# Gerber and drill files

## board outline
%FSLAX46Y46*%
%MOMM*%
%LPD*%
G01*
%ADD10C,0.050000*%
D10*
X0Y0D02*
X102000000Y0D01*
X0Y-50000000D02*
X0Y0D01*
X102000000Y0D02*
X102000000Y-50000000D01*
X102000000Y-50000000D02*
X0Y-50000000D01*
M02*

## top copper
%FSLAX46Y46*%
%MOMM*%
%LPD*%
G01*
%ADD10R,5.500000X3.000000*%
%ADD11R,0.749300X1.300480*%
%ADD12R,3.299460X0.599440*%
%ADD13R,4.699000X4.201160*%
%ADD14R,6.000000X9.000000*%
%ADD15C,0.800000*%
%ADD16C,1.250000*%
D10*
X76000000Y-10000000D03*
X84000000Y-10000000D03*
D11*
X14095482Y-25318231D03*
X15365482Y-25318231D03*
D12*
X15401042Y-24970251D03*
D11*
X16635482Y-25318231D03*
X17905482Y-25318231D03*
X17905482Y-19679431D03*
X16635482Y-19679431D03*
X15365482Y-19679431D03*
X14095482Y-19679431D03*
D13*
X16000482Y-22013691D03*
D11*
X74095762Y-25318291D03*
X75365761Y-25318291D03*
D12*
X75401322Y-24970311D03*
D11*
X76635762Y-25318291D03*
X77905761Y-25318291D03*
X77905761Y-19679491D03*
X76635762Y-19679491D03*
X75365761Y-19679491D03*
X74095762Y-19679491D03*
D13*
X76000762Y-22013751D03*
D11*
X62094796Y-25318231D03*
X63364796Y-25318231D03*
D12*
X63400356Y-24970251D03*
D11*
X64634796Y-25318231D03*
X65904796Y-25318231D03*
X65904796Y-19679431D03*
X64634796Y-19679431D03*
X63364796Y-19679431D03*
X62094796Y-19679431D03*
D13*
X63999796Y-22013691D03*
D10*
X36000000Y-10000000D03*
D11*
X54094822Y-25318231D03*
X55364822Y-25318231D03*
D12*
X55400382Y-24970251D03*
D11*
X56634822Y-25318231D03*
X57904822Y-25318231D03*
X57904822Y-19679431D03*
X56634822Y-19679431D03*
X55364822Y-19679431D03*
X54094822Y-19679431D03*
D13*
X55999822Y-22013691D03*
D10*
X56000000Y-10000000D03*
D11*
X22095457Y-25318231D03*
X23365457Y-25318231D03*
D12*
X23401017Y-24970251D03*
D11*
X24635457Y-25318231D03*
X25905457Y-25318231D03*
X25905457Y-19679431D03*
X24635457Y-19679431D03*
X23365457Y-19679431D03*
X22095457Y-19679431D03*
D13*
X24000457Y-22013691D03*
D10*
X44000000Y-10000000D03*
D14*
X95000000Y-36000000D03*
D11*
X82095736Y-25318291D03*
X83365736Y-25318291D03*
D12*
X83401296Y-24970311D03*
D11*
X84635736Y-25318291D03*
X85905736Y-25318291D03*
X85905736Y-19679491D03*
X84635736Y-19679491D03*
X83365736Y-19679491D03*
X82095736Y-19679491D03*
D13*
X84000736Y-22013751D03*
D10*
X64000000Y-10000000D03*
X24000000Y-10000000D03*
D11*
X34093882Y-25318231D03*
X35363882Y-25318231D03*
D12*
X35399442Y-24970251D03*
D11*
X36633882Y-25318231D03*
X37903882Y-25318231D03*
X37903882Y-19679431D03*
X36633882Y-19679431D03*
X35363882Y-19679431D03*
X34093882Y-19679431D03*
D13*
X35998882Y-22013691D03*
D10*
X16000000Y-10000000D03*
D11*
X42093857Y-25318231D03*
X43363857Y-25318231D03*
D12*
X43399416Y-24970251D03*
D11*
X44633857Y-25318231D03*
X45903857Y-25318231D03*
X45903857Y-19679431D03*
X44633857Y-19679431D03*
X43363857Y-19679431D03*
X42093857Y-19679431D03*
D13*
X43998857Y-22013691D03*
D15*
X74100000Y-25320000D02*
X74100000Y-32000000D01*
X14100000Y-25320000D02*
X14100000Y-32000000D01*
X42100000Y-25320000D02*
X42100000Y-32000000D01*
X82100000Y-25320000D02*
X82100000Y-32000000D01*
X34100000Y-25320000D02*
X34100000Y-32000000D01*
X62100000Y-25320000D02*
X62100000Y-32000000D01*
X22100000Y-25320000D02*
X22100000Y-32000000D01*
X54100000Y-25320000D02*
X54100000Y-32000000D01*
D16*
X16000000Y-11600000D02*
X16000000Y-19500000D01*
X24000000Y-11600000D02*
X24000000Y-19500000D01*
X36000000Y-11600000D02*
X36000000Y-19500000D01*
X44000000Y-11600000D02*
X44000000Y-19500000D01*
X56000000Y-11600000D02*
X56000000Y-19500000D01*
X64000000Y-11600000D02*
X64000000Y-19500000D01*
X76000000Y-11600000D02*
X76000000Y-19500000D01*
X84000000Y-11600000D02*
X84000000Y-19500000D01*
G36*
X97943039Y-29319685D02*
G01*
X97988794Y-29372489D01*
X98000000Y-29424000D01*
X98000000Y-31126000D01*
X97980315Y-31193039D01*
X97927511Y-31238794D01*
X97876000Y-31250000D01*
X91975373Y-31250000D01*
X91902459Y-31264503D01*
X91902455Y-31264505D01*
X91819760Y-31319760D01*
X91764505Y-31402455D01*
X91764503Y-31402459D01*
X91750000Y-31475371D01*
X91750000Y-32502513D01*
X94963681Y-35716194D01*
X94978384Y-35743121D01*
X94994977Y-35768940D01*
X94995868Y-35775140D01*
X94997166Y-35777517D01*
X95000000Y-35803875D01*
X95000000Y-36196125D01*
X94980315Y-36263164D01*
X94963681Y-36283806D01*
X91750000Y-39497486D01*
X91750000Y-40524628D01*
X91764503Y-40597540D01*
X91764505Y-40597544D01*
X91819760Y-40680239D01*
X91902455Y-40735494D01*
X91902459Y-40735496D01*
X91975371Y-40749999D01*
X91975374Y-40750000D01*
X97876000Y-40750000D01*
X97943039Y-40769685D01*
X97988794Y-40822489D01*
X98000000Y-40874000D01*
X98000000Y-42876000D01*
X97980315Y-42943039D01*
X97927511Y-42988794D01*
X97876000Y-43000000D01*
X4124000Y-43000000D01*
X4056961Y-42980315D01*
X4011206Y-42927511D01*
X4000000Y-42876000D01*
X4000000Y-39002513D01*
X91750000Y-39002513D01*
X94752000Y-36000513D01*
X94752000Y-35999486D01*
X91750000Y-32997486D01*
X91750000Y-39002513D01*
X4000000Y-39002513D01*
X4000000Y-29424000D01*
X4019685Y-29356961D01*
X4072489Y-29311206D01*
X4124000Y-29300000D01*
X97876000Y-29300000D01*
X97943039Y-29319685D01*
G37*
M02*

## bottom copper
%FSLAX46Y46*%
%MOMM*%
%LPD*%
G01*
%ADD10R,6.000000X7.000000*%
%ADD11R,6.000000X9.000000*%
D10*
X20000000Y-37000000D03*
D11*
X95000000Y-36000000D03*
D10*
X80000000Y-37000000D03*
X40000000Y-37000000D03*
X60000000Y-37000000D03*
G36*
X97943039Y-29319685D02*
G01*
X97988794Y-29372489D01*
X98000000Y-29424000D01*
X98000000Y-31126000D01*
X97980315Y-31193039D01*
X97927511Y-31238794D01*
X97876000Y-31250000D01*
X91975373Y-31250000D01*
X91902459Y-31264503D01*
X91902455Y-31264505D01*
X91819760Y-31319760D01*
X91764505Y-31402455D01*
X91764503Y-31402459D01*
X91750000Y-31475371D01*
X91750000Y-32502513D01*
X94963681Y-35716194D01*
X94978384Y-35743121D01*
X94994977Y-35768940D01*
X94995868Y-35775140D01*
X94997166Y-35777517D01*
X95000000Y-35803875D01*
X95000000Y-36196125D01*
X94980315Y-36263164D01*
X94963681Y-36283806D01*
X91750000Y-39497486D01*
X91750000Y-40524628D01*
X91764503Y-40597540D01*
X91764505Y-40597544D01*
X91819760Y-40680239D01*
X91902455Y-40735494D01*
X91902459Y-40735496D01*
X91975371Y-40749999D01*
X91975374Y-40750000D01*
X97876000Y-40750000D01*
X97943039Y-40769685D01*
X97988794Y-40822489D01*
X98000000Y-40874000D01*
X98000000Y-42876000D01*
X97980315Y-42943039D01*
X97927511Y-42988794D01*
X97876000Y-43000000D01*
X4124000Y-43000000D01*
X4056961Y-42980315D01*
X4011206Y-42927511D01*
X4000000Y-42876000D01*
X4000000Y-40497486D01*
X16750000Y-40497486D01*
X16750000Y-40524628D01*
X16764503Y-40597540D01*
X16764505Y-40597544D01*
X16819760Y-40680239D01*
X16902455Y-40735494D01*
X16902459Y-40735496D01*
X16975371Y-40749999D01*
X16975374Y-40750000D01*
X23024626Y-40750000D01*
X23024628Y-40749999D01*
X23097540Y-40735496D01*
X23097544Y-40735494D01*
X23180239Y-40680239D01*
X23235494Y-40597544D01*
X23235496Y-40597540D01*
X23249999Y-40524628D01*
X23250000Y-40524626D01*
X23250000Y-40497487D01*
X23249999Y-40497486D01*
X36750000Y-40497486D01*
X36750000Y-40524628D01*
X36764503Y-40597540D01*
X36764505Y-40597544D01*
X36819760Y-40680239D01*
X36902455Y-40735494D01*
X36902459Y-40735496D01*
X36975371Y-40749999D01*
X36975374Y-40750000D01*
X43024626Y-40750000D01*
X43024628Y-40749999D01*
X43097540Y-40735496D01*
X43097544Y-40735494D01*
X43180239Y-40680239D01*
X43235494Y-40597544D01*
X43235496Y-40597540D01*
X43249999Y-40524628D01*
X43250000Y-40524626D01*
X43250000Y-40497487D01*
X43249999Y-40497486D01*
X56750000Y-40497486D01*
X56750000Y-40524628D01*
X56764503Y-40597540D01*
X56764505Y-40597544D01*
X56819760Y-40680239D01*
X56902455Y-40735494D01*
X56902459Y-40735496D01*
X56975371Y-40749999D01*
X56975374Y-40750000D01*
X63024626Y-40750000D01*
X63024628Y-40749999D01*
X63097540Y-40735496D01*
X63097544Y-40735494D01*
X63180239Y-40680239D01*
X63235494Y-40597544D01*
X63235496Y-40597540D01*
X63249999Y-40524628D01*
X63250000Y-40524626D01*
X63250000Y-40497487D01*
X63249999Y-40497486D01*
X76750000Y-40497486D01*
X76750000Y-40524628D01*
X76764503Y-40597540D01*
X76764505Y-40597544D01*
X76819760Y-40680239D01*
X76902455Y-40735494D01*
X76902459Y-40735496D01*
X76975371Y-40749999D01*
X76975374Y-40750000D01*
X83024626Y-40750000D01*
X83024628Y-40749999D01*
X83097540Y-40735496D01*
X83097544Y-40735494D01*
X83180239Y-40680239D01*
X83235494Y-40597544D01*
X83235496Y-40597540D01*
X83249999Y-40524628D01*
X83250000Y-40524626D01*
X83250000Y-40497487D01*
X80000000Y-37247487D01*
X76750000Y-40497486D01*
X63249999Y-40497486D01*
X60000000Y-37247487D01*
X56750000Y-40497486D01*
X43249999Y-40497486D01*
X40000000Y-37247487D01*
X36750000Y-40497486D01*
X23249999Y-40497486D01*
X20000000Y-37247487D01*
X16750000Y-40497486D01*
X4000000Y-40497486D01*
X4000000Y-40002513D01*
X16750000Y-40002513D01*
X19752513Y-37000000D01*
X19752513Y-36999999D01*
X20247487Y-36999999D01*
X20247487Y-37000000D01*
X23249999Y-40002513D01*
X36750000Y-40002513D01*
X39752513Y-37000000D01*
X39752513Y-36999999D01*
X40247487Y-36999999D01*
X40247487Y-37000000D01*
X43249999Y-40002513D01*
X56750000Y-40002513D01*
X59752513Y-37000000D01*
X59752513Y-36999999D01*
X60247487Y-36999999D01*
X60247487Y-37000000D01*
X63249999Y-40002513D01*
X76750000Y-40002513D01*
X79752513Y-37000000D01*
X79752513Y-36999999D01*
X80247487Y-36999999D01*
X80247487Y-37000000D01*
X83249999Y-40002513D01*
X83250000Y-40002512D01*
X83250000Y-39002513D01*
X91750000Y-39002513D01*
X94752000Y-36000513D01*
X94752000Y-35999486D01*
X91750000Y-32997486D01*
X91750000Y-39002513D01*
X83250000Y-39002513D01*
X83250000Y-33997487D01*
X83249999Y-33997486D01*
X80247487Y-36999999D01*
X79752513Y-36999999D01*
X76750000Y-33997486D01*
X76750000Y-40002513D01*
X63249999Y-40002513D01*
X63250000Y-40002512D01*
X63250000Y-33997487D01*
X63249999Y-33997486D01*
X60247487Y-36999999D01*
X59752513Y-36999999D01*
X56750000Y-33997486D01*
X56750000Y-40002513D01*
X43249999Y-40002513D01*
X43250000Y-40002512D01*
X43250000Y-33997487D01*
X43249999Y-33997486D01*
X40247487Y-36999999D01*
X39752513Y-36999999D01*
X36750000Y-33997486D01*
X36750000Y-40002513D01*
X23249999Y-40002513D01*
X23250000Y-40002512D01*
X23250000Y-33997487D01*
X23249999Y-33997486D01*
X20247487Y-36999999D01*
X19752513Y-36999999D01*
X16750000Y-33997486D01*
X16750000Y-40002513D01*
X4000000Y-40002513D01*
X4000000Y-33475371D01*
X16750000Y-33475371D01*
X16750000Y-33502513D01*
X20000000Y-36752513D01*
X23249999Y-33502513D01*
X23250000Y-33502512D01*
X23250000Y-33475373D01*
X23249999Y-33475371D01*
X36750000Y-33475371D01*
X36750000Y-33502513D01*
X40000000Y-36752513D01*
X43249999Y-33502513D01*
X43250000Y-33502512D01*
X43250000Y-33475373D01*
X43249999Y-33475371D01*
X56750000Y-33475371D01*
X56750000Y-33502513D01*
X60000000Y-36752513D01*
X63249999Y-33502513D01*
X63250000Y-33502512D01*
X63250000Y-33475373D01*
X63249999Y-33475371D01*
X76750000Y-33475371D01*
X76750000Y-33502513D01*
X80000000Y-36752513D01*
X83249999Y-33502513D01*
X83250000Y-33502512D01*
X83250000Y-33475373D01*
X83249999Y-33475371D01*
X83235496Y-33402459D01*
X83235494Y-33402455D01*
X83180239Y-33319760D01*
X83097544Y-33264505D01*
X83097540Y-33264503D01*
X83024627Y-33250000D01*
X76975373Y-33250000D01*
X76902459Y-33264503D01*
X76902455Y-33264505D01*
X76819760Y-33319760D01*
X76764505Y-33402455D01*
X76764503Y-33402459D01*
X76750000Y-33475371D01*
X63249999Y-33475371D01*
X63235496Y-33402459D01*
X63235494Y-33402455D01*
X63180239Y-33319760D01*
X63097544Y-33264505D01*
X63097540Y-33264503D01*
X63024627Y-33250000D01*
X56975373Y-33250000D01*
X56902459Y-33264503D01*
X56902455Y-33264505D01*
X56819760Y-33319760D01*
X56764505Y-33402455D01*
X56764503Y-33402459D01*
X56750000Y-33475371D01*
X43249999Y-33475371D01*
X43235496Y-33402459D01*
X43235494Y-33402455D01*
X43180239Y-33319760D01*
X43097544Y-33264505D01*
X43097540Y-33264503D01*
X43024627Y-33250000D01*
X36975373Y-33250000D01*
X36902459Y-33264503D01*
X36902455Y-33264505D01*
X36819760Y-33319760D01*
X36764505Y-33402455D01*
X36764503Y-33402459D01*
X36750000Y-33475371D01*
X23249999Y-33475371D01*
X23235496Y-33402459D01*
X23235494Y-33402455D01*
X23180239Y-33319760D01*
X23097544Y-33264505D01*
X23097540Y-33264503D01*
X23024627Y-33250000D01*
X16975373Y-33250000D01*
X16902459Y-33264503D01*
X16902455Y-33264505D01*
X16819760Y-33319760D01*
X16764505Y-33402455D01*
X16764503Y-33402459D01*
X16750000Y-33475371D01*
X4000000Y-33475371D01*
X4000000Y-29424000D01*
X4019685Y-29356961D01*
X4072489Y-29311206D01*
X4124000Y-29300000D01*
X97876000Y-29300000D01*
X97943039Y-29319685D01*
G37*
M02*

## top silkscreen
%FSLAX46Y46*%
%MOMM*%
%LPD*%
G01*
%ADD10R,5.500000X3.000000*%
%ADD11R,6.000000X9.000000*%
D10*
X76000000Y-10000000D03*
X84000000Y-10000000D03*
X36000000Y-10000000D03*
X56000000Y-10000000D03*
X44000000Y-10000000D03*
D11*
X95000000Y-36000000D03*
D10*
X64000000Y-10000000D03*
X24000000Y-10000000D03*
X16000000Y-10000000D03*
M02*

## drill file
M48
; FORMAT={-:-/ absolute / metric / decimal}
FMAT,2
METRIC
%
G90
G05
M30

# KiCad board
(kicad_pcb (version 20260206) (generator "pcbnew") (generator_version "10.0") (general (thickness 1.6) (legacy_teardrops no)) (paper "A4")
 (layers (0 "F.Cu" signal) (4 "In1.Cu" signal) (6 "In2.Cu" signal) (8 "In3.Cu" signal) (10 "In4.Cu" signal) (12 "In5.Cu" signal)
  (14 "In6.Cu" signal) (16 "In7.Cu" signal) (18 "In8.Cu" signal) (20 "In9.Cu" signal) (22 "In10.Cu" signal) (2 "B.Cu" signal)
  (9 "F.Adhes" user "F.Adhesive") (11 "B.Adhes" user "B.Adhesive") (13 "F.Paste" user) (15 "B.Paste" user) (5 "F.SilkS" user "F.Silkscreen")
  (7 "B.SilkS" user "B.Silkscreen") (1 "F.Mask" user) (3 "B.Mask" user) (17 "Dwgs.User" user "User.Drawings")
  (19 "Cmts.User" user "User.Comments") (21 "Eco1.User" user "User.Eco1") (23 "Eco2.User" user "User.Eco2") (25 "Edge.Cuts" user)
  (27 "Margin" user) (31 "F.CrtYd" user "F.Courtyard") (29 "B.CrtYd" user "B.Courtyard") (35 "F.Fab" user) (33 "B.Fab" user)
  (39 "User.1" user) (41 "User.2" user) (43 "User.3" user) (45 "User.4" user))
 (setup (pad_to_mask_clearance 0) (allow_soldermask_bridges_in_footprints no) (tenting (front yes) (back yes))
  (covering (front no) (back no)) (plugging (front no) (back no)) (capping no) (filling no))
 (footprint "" (layer "F.Cu") (at 76 10)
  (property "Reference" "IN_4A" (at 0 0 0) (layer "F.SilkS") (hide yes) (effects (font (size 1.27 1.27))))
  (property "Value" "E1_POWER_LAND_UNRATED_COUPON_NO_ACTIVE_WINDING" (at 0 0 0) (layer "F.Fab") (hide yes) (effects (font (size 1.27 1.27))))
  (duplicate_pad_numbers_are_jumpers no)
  (pad "1" smd rect (at 0 0) (size 5.5 3)
   (layers "F.Cu" "F.Mask" "F.SilkS" "F.Adhes" "F.Paste" "F.CrtYd" "F.Fab") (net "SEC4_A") (thermal_bridge_angle 45)))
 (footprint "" (layer "F.Cu") (at 84 10)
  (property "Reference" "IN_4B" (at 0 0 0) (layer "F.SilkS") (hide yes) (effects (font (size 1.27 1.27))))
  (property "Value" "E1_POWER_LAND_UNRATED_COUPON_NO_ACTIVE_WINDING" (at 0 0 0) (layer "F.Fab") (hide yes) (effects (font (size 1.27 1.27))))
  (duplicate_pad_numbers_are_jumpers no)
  (pad "1" smd rect (at 0 0) (size 5.5 3)
   (layers "F.Cu" "F.Mask" "F.SilkS" "F.Adhes" "F.Paste" "F.CrtYd" "F.Fab") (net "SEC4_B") (thermal_bridge_angle 45)))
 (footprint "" (layer "F.Cu") (at 16 22.5)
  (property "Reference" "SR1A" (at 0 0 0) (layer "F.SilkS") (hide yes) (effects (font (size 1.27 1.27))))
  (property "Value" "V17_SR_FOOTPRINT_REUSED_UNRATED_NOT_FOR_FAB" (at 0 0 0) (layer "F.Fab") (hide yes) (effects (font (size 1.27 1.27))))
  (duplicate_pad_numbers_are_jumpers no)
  (pad "1" smd rect (at -1.904518 2.818231 90) (size 1.30048 0.7493) (layers "F.Cu" "F.Mask" "F.Paste") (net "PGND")
   (thermal_bridge_angle 45))
  (pad "2" smd rect (at -0.634518 2.818231 90) (size 1.30048 0.7493) (layers "F.Cu" "F.Mask" "F.Paste") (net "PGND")
   (thermal_bridge_angle 45))
  (pad "3" smd rect (at -0.598958 2.470251 90) (size 0.59944 3.29946) (layers "F.Cu" "F.Mask" "F.Paste") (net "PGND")
   (thermal_bridge_angle 45))
  (pad "3" smd rect (at 0.635482 2.818231 90) (size 1.30048 0.7493) (layers "F.Cu" "F.Mask" "F.Paste") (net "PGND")
   (thermal_bridge_angle 45))
  (pad "4" smd rect (at 1.905482 2.818231 90) (size 1.30048 0.7493) (layers "F.Cu" "F.Mask" "F.Paste") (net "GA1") (thermal_bridge_angle 45))
  (pad "5" smd rect (at 1.905482 -2.820569 270) (size 1.30048 0.7493) (layers "F.Cu" "F.Mask" "F.Paste") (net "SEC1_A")
   (thermal_bridge_angle 45))
  (pad "6" smd rect (at 0.635482 -2.820569 270) (size 1.30048 0.7493) (layers "F.Cu" "F.Mask" "F.Paste") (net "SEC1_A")
   (thermal_bridge_angle 45))
  (pad "7" smd rect (at -0.634518 -2.820569 270) (size 1.30048 0.7493) (layers "F.Cu" "F.Mask" "F.Paste") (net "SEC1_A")
   (thermal_bridge_angle 45))
  (pad "8" smd rect (at -1.904518 -2.820569 270) (size 1.30048 0.7493) (layers "F.Cu" "F.Mask" "F.Paste") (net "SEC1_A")
   (thermal_bridge_angle 45))
  (pad "8" smd rect (at 0.000482 -0.486309) (size 4.699 4.20116) (layers "F.Cu" "F.Mask" "F.Paste") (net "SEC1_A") (thermal_bridge_angle 45)))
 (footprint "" (layer "F.Cu") (at 76 22.5)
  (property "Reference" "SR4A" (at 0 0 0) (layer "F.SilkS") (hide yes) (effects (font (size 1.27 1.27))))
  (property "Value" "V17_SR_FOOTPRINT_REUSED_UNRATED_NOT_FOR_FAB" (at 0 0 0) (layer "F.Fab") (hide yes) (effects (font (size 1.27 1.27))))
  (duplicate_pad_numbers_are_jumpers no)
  (pad "1" smd rect (at -1.904238 2.818291 90) (size 1.30048 0.7493) (layers "F.Cu" "F.Mask" "F.Paste") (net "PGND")
   (thermal_bridge_angle 45))
  (pad "2" smd rect (at -0.634239 2.818291 90) (size 1.30048 0.7493) (layers "F.Cu" "F.Mask" "F.Paste") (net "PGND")
   (thermal_bridge_angle 45))
  (pad "3" smd rect (at -0.598678 2.470311 90) (size 0.59944 3.29946) (layers "F.Cu" "F.Mask" "F.Paste") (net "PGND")
   (thermal_bridge_angle 45))
  (pad "3" smd rect (at 0.635762 2.818291 90) (size 1.30048 0.7493) (layers "F.Cu" "F.Mask" "F.Paste") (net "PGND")
   (thermal_bridge_angle 45))
  (pad "4" smd rect (at 1.905761 2.818291 90) (size 1.30048 0.7493) (layers "F.Cu" "F.Mask" "F.Paste") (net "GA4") (thermal_bridge_angle 45))
  (pad "5" smd rect (at 1.905761 -2.820509 270) (size 1.30048 0.7493) (layers "F.Cu" "F.Mask" "F.Paste") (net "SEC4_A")
   (thermal_bridge_angle 45))
  (pad "6" smd rect (at 0.635762 -2.820509 270) (size 1.30048 0.7493) (layers "F.Cu" "F.Mask" "F.Paste") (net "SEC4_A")
   (thermal_bridge_angle 45))
  (pad "7" smd rect (at -0.634239 -2.820509 270) (size 1.30048 0.7493) (layers "F.Cu" "F.Mask" "F.Paste") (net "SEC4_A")
   (thermal_bridge_angle 45))
  (pad "8" smd rect (at -1.904238 -2.820509 270) (size 1.30048 0.7493) (layers "F.Cu" "F.Mask" "F.Paste") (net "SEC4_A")
   (thermal_bridge_angle 45))
  (pad "8" smd rect (at 0.000762 -0.486249) (size 4.699 4.20116) (layers "F.Cu" "F.Mask" "F.Paste") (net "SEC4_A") (thermal_bridge_angle 45)))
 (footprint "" (layer "F.Cu") (at 20 37)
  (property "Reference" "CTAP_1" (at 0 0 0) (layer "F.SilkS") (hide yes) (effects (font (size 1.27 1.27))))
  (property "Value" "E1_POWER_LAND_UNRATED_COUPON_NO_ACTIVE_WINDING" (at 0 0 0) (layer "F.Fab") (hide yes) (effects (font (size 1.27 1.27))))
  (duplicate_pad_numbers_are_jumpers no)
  (pad "1" smd rect (at 0 0) (size 6 7)
   (layers "B.Cu" "B.Mask" "B.SilkS" "B.Adhes" "B.Paste" "B.CrtYd" "B.Fab") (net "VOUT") (thermal_bridge_angle 45)))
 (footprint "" (layer "F.Cu") (at 64 22.5)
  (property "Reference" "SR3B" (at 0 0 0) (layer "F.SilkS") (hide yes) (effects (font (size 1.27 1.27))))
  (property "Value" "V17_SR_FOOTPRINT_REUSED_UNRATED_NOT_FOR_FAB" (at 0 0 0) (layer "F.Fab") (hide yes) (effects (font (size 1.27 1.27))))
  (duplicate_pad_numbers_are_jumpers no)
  (pad "1" smd rect (at -1.905204 2.818231 90) (size 1.30048 0.7493) (layers "F.Cu" "F.Mask" "F.Paste") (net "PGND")
   (thermal_bridge_angle 45))
  (pad "2" smd rect (at -0.635204 2.818231 90) (size 1.30048 0.7493) (layers "F.Cu" "F.Mask" "F.Paste") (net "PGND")
   (thermal_bridge_angle 45))
  (pad "3" smd rect (at -0.599644 2.470251 90) (size 0.59944 3.29946) (layers "F.Cu" "F.Mask" "F.Paste") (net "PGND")
   (thermal_bridge_angle 45))
  (pad "3" smd rect (at 0.634796 2.818231 90) (size 1.30048 0.7493) (layers "F.Cu" "F.Mask" "F.Paste") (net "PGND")
   (thermal_bridge_angle 45))
  (pad "4" smd rect (at 1.904796 2.818231 90) (size 1.30048 0.7493) (layers "F.Cu" "F.Mask" "F.Paste") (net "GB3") (thermal_bridge_angle 45))
  (pad "5" smd rect (at 1.904796 -2.820569 270) (size 1.30048 0.7493) (layers "F.Cu" "F.Mask" "F.Paste") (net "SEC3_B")
   (thermal_bridge_angle 45))
  (pad "6" smd rect (at 0.634796 -2.820569 270) (size 1.30048 0.7493) (layers "F.Cu" "F.Mask" "F.Paste") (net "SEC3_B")
   (thermal_bridge_angle 45))
  (pad "7" smd rect (at -0.635204 -2.820569 270) (size 1.30048 0.7493) (layers "F.Cu" "F.Mask" "F.Paste") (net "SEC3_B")
   (thermal_bridge_angle 45))
  (pad "8" smd rect (at -1.905204 -2.820569 270) (size 1.30048 0.7493) (layers "F.Cu" "F.Mask" "F.Paste") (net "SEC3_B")
   (thermal_bridge_angle 45))
  (pad "8" smd rect (at -0.000204 -0.486309) (size 4.699 4.20116) (layers "F.Cu" "F.Mask" "F.Paste") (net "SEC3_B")
   (thermal_bridge_angle 45)))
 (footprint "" (layer "F.Cu") (at 36 10)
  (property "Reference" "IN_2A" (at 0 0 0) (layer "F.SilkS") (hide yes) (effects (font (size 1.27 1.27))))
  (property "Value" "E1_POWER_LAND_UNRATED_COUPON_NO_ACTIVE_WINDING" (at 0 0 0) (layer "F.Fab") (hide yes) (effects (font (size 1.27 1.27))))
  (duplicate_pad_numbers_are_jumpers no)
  (pad "1" smd rect (at 0 0) (size 5.5 3)
   (layers "F.Cu" "F.Mask" "F.SilkS" "F.Adhes" "F.Paste" "F.CrtYd" "F.Fab") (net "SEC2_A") (thermal_bridge_angle 45)))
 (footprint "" (layer "F.Cu") (at 56 22.5)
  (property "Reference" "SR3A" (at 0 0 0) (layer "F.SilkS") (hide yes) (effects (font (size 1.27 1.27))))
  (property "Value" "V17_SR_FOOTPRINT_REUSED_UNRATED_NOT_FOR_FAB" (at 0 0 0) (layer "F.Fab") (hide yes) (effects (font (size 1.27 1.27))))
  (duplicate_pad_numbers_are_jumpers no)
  (pad "1" smd rect (at -1.905178 2.818231 90) (size 1.30048 0.7493) (layers "F.Cu" "F.Mask" "F.Paste") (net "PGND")
   (thermal_bridge_angle 45))
  (pad "2" smd rect (at -0.635178 2.818231 90) (size 1.30048 0.7493) (layers "F.Cu" "F.Mask" "F.Paste") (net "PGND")
   (thermal_bridge_angle 45))
  (pad "3" smd rect (at -0.599618 2.470251 90) (size 0.59944 3.29946) (layers "F.Cu" "F.Mask" "F.Paste") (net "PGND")
   (thermal_bridge_angle 45))
  (pad "3" smd rect (at 0.634822 2.818231 90) (size 1.30048 0.7493) (layers "F.Cu" "F.Mask" "F.Paste") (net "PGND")
   (thermal_bridge_angle 45))
  (pad "4" smd rect (at 1.904822 2.818231 90) (size 1.30048 0.7493) (layers "F.Cu" "F.Mask" "F.Paste") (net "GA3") (thermal_bridge_angle 45))
  (pad "5" smd rect (at 1.904822 -2.820569 270) (size 1.30048 0.7493) (layers "F.Cu" "F.Mask" "F.Paste") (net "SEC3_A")
   (thermal_bridge_angle 45))
  (pad "6" smd rect (at 0.634822 -2.820569 270) (size 1.30048 0.7493) (layers "F.Cu" "F.Mask" "F.Paste") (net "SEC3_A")
   (thermal_bridge_angle 45))
  (pad "7" smd rect (at -0.635178 -2.820569 270) (size 1.30048 0.7493) (layers "F.Cu" "F.Mask" "F.Paste") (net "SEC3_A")
   (thermal_bridge_angle 45))
  (pad "8" smd rect (at -1.905178 -2.820569 270) (size 1.30048 0.7493) (layers "F.Cu" "F.Mask" "F.Paste") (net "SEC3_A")
   (thermal_bridge_angle 45))
  (pad "8" smd rect (at -0.000178 -0.486309) (size 4.699 4.20116) (layers "F.Cu" "F.Mask" "F.Paste") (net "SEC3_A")
   (thermal_bridge_angle 45)))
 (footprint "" (layer "F.Cu") (at 56 10)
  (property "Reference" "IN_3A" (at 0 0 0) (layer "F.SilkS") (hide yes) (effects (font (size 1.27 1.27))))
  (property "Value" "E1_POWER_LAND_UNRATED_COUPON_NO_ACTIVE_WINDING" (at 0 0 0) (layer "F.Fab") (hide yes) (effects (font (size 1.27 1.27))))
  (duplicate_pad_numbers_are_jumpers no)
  (pad "1" smd rect (at 0 0) (size 5.5 3)
   (layers "F.Cu" "F.Mask" "F.SilkS" "F.Adhes" "F.Paste" "F.CrtYd" "F.Fab") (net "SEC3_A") (thermal_bridge_angle 45)))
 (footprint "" (layer "F.Cu") (at 95 36)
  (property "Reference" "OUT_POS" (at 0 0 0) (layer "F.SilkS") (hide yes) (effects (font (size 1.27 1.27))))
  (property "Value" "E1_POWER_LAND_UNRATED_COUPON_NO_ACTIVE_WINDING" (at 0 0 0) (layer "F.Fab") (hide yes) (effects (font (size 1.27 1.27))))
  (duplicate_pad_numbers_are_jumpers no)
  (pad "1" smd rect (at 0 0) (size 6 9)
   (layers "B.Cu" "B.Mask" "B.SilkS" "B.Adhes" "B.Paste" "B.CrtYd" "B.Fab") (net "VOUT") (thermal_bridge_angle 45)))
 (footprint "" (layer "F.Cu") (at 24 22.5)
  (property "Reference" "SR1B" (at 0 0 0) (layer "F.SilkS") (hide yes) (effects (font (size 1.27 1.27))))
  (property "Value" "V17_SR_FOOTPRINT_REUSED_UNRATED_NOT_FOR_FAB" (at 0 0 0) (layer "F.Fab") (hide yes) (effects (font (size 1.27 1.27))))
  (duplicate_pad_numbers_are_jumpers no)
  (pad "1" smd rect (at -1.904543 2.818231 90) (size 1.30048 0.7493) (layers "F.Cu" "F.Mask" "F.Paste") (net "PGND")
   (thermal_bridge_angle 45))
  (pad "2" smd rect (at -0.634543 2.818231 90) (size 1.30048 0.7493) (layers "F.Cu" "F.Mask" "F.Paste") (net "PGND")
   (thermal_bridge_angle 45))
  (pad "3" smd rect (at -0.598983 2.470251 90) (size 0.59944 3.29946) (layers "F.Cu" "F.Mask" "F.Paste") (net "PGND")
   (thermal_bridge_angle 45))
  (pad "3" smd rect (at 0.635457 2.818231 90) (size 1.30048 0.7493) (layers "F.Cu" "F.Mask" "F.Paste") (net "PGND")
   (thermal_bridge_angle 45))
  (pad "4" smd rect (at 1.905457 2.818231 90) (size 1.30048 0.7493) (layers "F.Cu" "F.Mask" "F.Paste") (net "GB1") (thermal_bridge_angle 45))
  (pad "5" smd rect (at 1.905457 -2.820569 270) (size 1.30048 0.7493) (layers "F.Cu" "F.Mask" "F.Paste") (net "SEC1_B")
   (thermal_bridge_angle 45))
  (pad "6" smd rect (at 0.635457 -2.820569 270) (size 1.30048 0.7493) (layers "F.Cu" "F.Mask" "F.Paste") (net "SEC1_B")
   (thermal_bridge_angle 45))
  (pad "7" smd rect (at -0.634543 -2.820569 270) (size 1.30048 0.7493) (layers "F.Cu" "F.Mask" "F.Paste") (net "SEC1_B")
   (thermal_bridge_angle 45))
  (pad "8" smd rect (at -1.904543 -2.820569 270) (size 1.30048 0.7493) (layers "F.Cu" "F.Mask" "F.Paste") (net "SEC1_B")
   (thermal_bridge_angle 45))
  (pad "8" smd rect (at 0.000457 -0.486309) (size 4.699 4.20116) (layers "F.Cu" "F.Mask" "F.Paste") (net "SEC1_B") (thermal_bridge_angle 45)))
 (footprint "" (layer "F.Cu") (at 80 37)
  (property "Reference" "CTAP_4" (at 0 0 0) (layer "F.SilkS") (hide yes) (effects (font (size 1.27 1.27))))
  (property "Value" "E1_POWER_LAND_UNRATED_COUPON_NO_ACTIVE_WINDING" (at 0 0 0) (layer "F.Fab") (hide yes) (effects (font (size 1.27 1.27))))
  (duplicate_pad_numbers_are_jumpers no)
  (pad "1" smd rect (at 0 0) (size 6 7)
   (layers "B.Cu" "B.Mask" "B.SilkS" "B.Adhes" "B.Paste" "B.CrtYd" "B.Fab") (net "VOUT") (thermal_bridge_angle 45)))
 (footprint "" (layer "F.Cu") (at 44 10)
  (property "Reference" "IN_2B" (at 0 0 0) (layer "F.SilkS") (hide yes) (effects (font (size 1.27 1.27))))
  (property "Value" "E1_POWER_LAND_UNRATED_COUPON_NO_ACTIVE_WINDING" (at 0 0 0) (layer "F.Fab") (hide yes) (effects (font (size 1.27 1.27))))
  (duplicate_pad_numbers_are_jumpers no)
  (pad "1" smd rect (at 0 0) (size 5.5 3)
   (layers "F.Cu" "F.Mask" "F.SilkS" "F.Adhes" "F.Paste" "F.CrtYd" "F.Fab") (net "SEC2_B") (thermal_bridge_angle 45)))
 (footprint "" (layer "F.Cu") (at 40 37)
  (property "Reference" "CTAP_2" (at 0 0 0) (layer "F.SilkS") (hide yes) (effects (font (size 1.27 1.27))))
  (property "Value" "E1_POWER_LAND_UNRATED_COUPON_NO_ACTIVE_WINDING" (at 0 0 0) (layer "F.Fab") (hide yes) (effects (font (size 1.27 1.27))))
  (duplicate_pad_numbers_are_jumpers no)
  (pad "1" smd rect (at 0 0) (size 6 7)
   (layers "B.Cu" "B.Mask" "B.SilkS" "B.Adhes" "B.Paste" "B.CrtYd" "B.Fab") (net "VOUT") (thermal_bridge_angle 45)))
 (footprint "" (layer "F.Cu") (at 95 36)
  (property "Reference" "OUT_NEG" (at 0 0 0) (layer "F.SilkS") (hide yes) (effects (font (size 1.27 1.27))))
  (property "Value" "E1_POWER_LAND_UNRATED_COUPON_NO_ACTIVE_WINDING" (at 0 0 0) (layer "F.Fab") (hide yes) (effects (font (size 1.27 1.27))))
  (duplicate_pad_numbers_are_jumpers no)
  (pad "1" smd rect (at 0 0) (size 6 9)
   (layers "F.Cu" "F.Mask" "F.SilkS" "F.Adhes" "F.Paste" "F.CrtYd" "F.Fab") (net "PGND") (thermal_bridge_angle 45)))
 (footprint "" (layer "F.Cu") (at 84 22.5)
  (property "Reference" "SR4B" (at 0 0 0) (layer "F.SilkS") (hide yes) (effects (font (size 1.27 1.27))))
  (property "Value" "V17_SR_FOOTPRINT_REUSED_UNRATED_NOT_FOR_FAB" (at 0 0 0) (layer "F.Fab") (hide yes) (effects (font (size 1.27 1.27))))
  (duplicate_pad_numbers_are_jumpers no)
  (pad "1" smd rect (at -1.904264 2.818291 90) (size 1.30048 0.7493) (layers "F.Cu" "F.Mask" "F.Paste") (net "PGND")
   (thermal_bridge_angle 45))
  (pad "2" smd rect (at -0.634264 2.818291 90) (size 1.30048 0.7493) (layers "F.Cu" "F.Mask" "F.Paste") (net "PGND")
   (thermal_bridge_angle 45))
  (pad "3" smd rect (at -0.598704 2.470311 90) (size 0.59944 3.29946) (layers "F.Cu" "F.Mask" "F.Paste") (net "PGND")
   (thermal_bridge_angle 45))
  (pad "3" smd rect (at 0.635736 2.818291 90) (size 1.30048 0.7493) (layers "F.Cu" "F.Mask" "F.Paste") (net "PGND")
   (thermal_bridge_angle 45))
  (pad "4" smd rect (at 1.905736 2.818291 90) (size 1.30048 0.7493) (layers "F.Cu" "F.Mask" "F.Paste") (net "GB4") (thermal_bridge_angle 45))
  (pad "5" smd rect (at 1.905736 -2.820509 270) (size 1.30048 0.7493) (layers "F.Cu" "F.Mask" "F.Paste") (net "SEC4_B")
   (thermal_bridge_angle 45))
  (pad "6" smd rect (at 0.635736 -2.820509 270) (size 1.30048 0.7493) (layers "F.Cu" "F.Mask" "F.Paste") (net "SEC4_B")
   (thermal_bridge_angle 45))
  (pad "7" smd rect (at -0.634264 -2.820509 270) (size 1.30048 0.7493) (layers "F.Cu" "F.Mask" "F.Paste") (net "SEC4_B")
   (thermal_bridge_angle 45))
  (pad "8" smd rect (at -1.904264 -2.820509 270) (size 1.30048 0.7493) (layers "F.Cu" "F.Mask" "F.Paste") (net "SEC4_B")
   (thermal_bridge_angle 45))
  (pad "8" smd rect (at 0.000736 -0.486249) (size 4.699 4.20116) (layers "F.Cu" "F.Mask" "F.Paste") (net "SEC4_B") (thermal_bridge_angle 45)))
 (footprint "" (layer "F.Cu") (at 64 10)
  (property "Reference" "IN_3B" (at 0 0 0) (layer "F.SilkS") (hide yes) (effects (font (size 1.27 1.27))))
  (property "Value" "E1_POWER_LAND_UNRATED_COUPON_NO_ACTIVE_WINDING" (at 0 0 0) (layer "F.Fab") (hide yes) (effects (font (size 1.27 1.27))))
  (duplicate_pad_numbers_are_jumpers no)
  (pad "1" smd rect (at 0 0) (size 5.5 3)
   (layers "F.Cu" "F.Mask" "F.SilkS" "F.Adhes" "F.Paste" "F.CrtYd" "F.Fab") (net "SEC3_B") (thermal_bridge_angle 45)))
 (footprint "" (layer "F.Cu") (at 24 10)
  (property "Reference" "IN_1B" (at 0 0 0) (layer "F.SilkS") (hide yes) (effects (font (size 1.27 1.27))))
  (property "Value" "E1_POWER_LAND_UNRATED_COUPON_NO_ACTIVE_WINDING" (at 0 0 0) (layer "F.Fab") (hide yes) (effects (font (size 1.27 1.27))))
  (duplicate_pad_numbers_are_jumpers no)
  (pad "1" smd rect (at 0 0) (size 5.5 3)
   (layers "F.Cu" "F.Mask" "F.SilkS" "F.Adhes" "F.Paste" "F.CrtYd" "F.Fab") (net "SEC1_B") (thermal_bridge_angle 45)))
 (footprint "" (layer "F.Cu") (at 36 22.5)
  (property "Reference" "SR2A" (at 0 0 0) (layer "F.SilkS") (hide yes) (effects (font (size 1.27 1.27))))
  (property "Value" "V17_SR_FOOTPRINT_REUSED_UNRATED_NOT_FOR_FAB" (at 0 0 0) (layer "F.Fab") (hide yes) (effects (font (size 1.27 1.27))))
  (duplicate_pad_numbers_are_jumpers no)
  (pad "1" smd rect (at -1.906118 2.818231 90) (size 1.30048 0.7493) (layers "F.Cu" "F.Mask" "F.Paste") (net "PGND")
   (thermal_bridge_angle 45))
  (pad "2" smd rect (at -0.636118 2.818231 90) (size 1.30048 0.7493) (layers "F.Cu" "F.Mask" "F.Paste") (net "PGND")
   (thermal_bridge_angle 45))
  (pad "3" smd rect (at -0.600558 2.470251 90) (size 0.59944 3.29946) (layers "F.Cu" "F.Mask" "F.Paste") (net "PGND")
   (thermal_bridge_angle 45))
  (pad "3" smd rect (at 0.633882 2.818231 90) (size 1.30048 0.7493) (layers "F.Cu" "F.Mask" "F.Paste") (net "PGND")
   (thermal_bridge_angle 45))
  (pad "4" smd rect (at 1.903882 2.818231 90) (size 1.30048 0.7493) (layers "F.Cu" "F.Mask" "F.Paste") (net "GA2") (thermal_bridge_angle 45))
  (pad "5" smd rect (at 1.903882 -2.820569 270) (size 1.30048 0.7493) (layers "F.Cu" "F.Mask" "F.Paste") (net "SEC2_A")
   (thermal_bridge_angle 45))
  (pad "6" smd rect (at 0.633882 -2.820569 270) (size 1.30048 0.7493) (layers "F.Cu" "F.Mask" "F.Paste") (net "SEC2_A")
   (thermal_bridge_angle 45))
  (pad "7" smd rect (at -0.636118 -2.820569 270) (size 1.30048 0.7493) (layers "F.Cu" "F.Mask" "F.Paste") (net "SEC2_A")
   (thermal_bridge_angle 45))
  (pad "8" smd rect (at -1.906118 -2.820569 270) (size 1.30048 0.7493) (layers "F.Cu" "F.Mask" "F.Paste") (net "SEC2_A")
   (thermal_bridge_angle 45))
  (pad "8" smd rect (at -0.001118 -0.486309) (size 4.699 4.20116) (layers "F.Cu" "F.Mask" "F.Paste") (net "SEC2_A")
   (thermal_bridge_angle 45)))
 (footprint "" (layer "F.Cu") (at 16 10)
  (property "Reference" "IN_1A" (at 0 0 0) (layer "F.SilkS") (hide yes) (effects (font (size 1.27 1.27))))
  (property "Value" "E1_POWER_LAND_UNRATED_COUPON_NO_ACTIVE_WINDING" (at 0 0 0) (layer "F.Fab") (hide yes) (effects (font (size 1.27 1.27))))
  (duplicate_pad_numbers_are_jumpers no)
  (pad "1" smd rect (at 0 0) (size 5.5 3)
   (layers "F.Cu" "F.Mask" "F.SilkS" "F.Adhes" "F.Paste" "F.CrtYd" "F.Fab") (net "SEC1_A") (thermal_bridge_angle 45)))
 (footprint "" (layer "F.Cu") (at 60 37)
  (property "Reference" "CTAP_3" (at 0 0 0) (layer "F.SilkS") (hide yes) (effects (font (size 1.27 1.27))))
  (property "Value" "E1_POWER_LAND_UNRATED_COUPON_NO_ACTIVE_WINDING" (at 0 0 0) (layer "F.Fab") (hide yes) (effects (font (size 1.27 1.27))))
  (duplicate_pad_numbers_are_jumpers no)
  (pad "1" smd rect (at 0 0) (size 6 7)
   (layers "B.Cu" "B.Mask" "B.SilkS" "B.Adhes" "B.Paste" "B.CrtYd" "B.Fab") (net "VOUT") (thermal_bridge_angle 45)))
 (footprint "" (layer "F.Cu") (at 44 22.5)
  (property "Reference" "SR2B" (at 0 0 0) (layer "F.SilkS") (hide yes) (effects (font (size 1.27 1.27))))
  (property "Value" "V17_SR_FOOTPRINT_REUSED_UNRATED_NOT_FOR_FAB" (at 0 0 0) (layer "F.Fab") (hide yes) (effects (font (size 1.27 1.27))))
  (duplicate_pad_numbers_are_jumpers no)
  (pad "1" smd rect (at -1.906143 2.818231 90) (size 1.30048 0.7493) (layers "F.Cu" "F.Mask" "F.Paste") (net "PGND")
   (thermal_bridge_angle 45))
  (pad "2" smd rect (at -0.636143 2.818231 90) (size 1.30048 0.7493) (layers "F.Cu" "F.Mask" "F.Paste") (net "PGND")
   (thermal_bridge_angle 45))
  (pad "3" smd rect (at -0.600584 2.470251 90) (size 0.59944 3.29946) (layers "F.Cu" "F.Mask" "F.Paste") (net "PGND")
   (thermal_bridge_angle 45))
  (pad "3" smd rect (at 0.633857 2.818231 90) (size 1.30048 0.7493) (layers "F.Cu" "F.Mask" "F.Paste") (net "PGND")
   (thermal_bridge_angle 45))
  (pad "4" smd rect (at 1.903857 2.818231 90) (size 1.30048 0.7493) (layers "F.Cu" "F.Mask" "F.Paste") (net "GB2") (thermal_bridge_angle 45))
  (pad "5" smd rect (at 1.903857 -2.820569 270) (size 1.30048 0.7493) (layers "F.Cu" "F.Mask" "F.Paste") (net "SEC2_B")
   (thermal_bridge_angle 45))
  (pad "6" smd rect (at 0.633857 -2.820569 270) (size 1.30048 0.7493) (layers "F.Cu" "F.Mask" "F.Paste") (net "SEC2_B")
   (thermal_bridge_angle 45))
  (pad "7" smd rect (at -0.636143 -2.820569 270) (size 1.30048 0.7493) (layers "F.Cu" "F.Mask" "F.Paste") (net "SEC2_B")
   (thermal_bridge_angle 45))
  (pad "8" smd rect (at -1.906143 -2.820569 270) (size 1.30048 0.7493) (layers "F.Cu" "F.Mask" "F.Paste") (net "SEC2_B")
   (thermal_bridge_angle 45))
  (pad "8" smd rect (at -0.001143 -0.486309) (size 4.699 4.20116) (layers "F.Cu" "F.Mask" "F.Paste") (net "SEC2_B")
   (thermal_bridge_angle 45)))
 (gr_line (start 0 0) (end 102 0) (stroke (width 0.05) (type default)) (layer "Edge.Cuts"))
 (gr_line (start 0 50) (end 0 0) (stroke (width 0.05) (type default)) (layer "Edge.Cuts"))
 (gr_line (start 102 0) (end 102 50) (stroke (width 0.05) (type default)) (layer "Edge.Cuts"))
 (gr_line (start 102 50) (end 0 50) (stroke (width 0.05) (type default)) (layer "Edge.Cuts"))
 (segment (start 74.1 25.32) (end 74.1 32) (width 0.8) (layer "F.Cu") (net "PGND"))
 (segment (start 14.1 25.32) (end 14.1 32) (width 0.8) (layer "F.Cu") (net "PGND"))
 (segment (start 42.1 25.32) (end 42.1 32) (width 0.8) (layer "F.Cu") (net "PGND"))
 (segment (start 82.1 25.32) (end 82.1 32) (width 0.8) (layer "F.Cu") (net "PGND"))
 (segment (start 34.1 25.32) (end 34.1 32) (width 0.8) (layer "F.Cu") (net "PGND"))
 (segment (start 62.1 25.32) (end 62.1 32) (width 0.8) (layer "F.Cu") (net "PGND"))
 (segment (start 22.1 25.32) (end 22.1 32) (width 0.8) (layer "F.Cu") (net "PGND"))
 (segment (start 54.1 25.32) (end 54.1 32) (width 0.8) (layer "F.Cu") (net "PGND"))
 (segment (start 16 11.6) (end 16 19.5) (width 1.25) (layer "F.Cu") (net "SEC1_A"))
 (segment (start 24 11.6) (end 24 19.5) (width 1.25) (layer "F.Cu") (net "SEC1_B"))
 (segment (start 36 11.6) (end 36 19.5) (width 1.25) (layer "F.Cu") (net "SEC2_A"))
 (segment (start 44 11.6) (end 44 19.5) (width 1.25) (layer "F.Cu") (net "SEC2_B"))
 (segment (start 56 11.6) (end 56 19.5) (width 1.25) (layer "F.Cu") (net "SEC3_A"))
 (segment (start 64 11.6) (end 64 19.5) (width 1.25) (layer "F.Cu") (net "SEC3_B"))
 (segment (start 76 11.6) (end 76 19.5) (width 1.25) (layer "F.Cu") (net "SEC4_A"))
 (segment (start 84 11.6) (end 84 19.5) (width 1.25) (layer "F.Cu") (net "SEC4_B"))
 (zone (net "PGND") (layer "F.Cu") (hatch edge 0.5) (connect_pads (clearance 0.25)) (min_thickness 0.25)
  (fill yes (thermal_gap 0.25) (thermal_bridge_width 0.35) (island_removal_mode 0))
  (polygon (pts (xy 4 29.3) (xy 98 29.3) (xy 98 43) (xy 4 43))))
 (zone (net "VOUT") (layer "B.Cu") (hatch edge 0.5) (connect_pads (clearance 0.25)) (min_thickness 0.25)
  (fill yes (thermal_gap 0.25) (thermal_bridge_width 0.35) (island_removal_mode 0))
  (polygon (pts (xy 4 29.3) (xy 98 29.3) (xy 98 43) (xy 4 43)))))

